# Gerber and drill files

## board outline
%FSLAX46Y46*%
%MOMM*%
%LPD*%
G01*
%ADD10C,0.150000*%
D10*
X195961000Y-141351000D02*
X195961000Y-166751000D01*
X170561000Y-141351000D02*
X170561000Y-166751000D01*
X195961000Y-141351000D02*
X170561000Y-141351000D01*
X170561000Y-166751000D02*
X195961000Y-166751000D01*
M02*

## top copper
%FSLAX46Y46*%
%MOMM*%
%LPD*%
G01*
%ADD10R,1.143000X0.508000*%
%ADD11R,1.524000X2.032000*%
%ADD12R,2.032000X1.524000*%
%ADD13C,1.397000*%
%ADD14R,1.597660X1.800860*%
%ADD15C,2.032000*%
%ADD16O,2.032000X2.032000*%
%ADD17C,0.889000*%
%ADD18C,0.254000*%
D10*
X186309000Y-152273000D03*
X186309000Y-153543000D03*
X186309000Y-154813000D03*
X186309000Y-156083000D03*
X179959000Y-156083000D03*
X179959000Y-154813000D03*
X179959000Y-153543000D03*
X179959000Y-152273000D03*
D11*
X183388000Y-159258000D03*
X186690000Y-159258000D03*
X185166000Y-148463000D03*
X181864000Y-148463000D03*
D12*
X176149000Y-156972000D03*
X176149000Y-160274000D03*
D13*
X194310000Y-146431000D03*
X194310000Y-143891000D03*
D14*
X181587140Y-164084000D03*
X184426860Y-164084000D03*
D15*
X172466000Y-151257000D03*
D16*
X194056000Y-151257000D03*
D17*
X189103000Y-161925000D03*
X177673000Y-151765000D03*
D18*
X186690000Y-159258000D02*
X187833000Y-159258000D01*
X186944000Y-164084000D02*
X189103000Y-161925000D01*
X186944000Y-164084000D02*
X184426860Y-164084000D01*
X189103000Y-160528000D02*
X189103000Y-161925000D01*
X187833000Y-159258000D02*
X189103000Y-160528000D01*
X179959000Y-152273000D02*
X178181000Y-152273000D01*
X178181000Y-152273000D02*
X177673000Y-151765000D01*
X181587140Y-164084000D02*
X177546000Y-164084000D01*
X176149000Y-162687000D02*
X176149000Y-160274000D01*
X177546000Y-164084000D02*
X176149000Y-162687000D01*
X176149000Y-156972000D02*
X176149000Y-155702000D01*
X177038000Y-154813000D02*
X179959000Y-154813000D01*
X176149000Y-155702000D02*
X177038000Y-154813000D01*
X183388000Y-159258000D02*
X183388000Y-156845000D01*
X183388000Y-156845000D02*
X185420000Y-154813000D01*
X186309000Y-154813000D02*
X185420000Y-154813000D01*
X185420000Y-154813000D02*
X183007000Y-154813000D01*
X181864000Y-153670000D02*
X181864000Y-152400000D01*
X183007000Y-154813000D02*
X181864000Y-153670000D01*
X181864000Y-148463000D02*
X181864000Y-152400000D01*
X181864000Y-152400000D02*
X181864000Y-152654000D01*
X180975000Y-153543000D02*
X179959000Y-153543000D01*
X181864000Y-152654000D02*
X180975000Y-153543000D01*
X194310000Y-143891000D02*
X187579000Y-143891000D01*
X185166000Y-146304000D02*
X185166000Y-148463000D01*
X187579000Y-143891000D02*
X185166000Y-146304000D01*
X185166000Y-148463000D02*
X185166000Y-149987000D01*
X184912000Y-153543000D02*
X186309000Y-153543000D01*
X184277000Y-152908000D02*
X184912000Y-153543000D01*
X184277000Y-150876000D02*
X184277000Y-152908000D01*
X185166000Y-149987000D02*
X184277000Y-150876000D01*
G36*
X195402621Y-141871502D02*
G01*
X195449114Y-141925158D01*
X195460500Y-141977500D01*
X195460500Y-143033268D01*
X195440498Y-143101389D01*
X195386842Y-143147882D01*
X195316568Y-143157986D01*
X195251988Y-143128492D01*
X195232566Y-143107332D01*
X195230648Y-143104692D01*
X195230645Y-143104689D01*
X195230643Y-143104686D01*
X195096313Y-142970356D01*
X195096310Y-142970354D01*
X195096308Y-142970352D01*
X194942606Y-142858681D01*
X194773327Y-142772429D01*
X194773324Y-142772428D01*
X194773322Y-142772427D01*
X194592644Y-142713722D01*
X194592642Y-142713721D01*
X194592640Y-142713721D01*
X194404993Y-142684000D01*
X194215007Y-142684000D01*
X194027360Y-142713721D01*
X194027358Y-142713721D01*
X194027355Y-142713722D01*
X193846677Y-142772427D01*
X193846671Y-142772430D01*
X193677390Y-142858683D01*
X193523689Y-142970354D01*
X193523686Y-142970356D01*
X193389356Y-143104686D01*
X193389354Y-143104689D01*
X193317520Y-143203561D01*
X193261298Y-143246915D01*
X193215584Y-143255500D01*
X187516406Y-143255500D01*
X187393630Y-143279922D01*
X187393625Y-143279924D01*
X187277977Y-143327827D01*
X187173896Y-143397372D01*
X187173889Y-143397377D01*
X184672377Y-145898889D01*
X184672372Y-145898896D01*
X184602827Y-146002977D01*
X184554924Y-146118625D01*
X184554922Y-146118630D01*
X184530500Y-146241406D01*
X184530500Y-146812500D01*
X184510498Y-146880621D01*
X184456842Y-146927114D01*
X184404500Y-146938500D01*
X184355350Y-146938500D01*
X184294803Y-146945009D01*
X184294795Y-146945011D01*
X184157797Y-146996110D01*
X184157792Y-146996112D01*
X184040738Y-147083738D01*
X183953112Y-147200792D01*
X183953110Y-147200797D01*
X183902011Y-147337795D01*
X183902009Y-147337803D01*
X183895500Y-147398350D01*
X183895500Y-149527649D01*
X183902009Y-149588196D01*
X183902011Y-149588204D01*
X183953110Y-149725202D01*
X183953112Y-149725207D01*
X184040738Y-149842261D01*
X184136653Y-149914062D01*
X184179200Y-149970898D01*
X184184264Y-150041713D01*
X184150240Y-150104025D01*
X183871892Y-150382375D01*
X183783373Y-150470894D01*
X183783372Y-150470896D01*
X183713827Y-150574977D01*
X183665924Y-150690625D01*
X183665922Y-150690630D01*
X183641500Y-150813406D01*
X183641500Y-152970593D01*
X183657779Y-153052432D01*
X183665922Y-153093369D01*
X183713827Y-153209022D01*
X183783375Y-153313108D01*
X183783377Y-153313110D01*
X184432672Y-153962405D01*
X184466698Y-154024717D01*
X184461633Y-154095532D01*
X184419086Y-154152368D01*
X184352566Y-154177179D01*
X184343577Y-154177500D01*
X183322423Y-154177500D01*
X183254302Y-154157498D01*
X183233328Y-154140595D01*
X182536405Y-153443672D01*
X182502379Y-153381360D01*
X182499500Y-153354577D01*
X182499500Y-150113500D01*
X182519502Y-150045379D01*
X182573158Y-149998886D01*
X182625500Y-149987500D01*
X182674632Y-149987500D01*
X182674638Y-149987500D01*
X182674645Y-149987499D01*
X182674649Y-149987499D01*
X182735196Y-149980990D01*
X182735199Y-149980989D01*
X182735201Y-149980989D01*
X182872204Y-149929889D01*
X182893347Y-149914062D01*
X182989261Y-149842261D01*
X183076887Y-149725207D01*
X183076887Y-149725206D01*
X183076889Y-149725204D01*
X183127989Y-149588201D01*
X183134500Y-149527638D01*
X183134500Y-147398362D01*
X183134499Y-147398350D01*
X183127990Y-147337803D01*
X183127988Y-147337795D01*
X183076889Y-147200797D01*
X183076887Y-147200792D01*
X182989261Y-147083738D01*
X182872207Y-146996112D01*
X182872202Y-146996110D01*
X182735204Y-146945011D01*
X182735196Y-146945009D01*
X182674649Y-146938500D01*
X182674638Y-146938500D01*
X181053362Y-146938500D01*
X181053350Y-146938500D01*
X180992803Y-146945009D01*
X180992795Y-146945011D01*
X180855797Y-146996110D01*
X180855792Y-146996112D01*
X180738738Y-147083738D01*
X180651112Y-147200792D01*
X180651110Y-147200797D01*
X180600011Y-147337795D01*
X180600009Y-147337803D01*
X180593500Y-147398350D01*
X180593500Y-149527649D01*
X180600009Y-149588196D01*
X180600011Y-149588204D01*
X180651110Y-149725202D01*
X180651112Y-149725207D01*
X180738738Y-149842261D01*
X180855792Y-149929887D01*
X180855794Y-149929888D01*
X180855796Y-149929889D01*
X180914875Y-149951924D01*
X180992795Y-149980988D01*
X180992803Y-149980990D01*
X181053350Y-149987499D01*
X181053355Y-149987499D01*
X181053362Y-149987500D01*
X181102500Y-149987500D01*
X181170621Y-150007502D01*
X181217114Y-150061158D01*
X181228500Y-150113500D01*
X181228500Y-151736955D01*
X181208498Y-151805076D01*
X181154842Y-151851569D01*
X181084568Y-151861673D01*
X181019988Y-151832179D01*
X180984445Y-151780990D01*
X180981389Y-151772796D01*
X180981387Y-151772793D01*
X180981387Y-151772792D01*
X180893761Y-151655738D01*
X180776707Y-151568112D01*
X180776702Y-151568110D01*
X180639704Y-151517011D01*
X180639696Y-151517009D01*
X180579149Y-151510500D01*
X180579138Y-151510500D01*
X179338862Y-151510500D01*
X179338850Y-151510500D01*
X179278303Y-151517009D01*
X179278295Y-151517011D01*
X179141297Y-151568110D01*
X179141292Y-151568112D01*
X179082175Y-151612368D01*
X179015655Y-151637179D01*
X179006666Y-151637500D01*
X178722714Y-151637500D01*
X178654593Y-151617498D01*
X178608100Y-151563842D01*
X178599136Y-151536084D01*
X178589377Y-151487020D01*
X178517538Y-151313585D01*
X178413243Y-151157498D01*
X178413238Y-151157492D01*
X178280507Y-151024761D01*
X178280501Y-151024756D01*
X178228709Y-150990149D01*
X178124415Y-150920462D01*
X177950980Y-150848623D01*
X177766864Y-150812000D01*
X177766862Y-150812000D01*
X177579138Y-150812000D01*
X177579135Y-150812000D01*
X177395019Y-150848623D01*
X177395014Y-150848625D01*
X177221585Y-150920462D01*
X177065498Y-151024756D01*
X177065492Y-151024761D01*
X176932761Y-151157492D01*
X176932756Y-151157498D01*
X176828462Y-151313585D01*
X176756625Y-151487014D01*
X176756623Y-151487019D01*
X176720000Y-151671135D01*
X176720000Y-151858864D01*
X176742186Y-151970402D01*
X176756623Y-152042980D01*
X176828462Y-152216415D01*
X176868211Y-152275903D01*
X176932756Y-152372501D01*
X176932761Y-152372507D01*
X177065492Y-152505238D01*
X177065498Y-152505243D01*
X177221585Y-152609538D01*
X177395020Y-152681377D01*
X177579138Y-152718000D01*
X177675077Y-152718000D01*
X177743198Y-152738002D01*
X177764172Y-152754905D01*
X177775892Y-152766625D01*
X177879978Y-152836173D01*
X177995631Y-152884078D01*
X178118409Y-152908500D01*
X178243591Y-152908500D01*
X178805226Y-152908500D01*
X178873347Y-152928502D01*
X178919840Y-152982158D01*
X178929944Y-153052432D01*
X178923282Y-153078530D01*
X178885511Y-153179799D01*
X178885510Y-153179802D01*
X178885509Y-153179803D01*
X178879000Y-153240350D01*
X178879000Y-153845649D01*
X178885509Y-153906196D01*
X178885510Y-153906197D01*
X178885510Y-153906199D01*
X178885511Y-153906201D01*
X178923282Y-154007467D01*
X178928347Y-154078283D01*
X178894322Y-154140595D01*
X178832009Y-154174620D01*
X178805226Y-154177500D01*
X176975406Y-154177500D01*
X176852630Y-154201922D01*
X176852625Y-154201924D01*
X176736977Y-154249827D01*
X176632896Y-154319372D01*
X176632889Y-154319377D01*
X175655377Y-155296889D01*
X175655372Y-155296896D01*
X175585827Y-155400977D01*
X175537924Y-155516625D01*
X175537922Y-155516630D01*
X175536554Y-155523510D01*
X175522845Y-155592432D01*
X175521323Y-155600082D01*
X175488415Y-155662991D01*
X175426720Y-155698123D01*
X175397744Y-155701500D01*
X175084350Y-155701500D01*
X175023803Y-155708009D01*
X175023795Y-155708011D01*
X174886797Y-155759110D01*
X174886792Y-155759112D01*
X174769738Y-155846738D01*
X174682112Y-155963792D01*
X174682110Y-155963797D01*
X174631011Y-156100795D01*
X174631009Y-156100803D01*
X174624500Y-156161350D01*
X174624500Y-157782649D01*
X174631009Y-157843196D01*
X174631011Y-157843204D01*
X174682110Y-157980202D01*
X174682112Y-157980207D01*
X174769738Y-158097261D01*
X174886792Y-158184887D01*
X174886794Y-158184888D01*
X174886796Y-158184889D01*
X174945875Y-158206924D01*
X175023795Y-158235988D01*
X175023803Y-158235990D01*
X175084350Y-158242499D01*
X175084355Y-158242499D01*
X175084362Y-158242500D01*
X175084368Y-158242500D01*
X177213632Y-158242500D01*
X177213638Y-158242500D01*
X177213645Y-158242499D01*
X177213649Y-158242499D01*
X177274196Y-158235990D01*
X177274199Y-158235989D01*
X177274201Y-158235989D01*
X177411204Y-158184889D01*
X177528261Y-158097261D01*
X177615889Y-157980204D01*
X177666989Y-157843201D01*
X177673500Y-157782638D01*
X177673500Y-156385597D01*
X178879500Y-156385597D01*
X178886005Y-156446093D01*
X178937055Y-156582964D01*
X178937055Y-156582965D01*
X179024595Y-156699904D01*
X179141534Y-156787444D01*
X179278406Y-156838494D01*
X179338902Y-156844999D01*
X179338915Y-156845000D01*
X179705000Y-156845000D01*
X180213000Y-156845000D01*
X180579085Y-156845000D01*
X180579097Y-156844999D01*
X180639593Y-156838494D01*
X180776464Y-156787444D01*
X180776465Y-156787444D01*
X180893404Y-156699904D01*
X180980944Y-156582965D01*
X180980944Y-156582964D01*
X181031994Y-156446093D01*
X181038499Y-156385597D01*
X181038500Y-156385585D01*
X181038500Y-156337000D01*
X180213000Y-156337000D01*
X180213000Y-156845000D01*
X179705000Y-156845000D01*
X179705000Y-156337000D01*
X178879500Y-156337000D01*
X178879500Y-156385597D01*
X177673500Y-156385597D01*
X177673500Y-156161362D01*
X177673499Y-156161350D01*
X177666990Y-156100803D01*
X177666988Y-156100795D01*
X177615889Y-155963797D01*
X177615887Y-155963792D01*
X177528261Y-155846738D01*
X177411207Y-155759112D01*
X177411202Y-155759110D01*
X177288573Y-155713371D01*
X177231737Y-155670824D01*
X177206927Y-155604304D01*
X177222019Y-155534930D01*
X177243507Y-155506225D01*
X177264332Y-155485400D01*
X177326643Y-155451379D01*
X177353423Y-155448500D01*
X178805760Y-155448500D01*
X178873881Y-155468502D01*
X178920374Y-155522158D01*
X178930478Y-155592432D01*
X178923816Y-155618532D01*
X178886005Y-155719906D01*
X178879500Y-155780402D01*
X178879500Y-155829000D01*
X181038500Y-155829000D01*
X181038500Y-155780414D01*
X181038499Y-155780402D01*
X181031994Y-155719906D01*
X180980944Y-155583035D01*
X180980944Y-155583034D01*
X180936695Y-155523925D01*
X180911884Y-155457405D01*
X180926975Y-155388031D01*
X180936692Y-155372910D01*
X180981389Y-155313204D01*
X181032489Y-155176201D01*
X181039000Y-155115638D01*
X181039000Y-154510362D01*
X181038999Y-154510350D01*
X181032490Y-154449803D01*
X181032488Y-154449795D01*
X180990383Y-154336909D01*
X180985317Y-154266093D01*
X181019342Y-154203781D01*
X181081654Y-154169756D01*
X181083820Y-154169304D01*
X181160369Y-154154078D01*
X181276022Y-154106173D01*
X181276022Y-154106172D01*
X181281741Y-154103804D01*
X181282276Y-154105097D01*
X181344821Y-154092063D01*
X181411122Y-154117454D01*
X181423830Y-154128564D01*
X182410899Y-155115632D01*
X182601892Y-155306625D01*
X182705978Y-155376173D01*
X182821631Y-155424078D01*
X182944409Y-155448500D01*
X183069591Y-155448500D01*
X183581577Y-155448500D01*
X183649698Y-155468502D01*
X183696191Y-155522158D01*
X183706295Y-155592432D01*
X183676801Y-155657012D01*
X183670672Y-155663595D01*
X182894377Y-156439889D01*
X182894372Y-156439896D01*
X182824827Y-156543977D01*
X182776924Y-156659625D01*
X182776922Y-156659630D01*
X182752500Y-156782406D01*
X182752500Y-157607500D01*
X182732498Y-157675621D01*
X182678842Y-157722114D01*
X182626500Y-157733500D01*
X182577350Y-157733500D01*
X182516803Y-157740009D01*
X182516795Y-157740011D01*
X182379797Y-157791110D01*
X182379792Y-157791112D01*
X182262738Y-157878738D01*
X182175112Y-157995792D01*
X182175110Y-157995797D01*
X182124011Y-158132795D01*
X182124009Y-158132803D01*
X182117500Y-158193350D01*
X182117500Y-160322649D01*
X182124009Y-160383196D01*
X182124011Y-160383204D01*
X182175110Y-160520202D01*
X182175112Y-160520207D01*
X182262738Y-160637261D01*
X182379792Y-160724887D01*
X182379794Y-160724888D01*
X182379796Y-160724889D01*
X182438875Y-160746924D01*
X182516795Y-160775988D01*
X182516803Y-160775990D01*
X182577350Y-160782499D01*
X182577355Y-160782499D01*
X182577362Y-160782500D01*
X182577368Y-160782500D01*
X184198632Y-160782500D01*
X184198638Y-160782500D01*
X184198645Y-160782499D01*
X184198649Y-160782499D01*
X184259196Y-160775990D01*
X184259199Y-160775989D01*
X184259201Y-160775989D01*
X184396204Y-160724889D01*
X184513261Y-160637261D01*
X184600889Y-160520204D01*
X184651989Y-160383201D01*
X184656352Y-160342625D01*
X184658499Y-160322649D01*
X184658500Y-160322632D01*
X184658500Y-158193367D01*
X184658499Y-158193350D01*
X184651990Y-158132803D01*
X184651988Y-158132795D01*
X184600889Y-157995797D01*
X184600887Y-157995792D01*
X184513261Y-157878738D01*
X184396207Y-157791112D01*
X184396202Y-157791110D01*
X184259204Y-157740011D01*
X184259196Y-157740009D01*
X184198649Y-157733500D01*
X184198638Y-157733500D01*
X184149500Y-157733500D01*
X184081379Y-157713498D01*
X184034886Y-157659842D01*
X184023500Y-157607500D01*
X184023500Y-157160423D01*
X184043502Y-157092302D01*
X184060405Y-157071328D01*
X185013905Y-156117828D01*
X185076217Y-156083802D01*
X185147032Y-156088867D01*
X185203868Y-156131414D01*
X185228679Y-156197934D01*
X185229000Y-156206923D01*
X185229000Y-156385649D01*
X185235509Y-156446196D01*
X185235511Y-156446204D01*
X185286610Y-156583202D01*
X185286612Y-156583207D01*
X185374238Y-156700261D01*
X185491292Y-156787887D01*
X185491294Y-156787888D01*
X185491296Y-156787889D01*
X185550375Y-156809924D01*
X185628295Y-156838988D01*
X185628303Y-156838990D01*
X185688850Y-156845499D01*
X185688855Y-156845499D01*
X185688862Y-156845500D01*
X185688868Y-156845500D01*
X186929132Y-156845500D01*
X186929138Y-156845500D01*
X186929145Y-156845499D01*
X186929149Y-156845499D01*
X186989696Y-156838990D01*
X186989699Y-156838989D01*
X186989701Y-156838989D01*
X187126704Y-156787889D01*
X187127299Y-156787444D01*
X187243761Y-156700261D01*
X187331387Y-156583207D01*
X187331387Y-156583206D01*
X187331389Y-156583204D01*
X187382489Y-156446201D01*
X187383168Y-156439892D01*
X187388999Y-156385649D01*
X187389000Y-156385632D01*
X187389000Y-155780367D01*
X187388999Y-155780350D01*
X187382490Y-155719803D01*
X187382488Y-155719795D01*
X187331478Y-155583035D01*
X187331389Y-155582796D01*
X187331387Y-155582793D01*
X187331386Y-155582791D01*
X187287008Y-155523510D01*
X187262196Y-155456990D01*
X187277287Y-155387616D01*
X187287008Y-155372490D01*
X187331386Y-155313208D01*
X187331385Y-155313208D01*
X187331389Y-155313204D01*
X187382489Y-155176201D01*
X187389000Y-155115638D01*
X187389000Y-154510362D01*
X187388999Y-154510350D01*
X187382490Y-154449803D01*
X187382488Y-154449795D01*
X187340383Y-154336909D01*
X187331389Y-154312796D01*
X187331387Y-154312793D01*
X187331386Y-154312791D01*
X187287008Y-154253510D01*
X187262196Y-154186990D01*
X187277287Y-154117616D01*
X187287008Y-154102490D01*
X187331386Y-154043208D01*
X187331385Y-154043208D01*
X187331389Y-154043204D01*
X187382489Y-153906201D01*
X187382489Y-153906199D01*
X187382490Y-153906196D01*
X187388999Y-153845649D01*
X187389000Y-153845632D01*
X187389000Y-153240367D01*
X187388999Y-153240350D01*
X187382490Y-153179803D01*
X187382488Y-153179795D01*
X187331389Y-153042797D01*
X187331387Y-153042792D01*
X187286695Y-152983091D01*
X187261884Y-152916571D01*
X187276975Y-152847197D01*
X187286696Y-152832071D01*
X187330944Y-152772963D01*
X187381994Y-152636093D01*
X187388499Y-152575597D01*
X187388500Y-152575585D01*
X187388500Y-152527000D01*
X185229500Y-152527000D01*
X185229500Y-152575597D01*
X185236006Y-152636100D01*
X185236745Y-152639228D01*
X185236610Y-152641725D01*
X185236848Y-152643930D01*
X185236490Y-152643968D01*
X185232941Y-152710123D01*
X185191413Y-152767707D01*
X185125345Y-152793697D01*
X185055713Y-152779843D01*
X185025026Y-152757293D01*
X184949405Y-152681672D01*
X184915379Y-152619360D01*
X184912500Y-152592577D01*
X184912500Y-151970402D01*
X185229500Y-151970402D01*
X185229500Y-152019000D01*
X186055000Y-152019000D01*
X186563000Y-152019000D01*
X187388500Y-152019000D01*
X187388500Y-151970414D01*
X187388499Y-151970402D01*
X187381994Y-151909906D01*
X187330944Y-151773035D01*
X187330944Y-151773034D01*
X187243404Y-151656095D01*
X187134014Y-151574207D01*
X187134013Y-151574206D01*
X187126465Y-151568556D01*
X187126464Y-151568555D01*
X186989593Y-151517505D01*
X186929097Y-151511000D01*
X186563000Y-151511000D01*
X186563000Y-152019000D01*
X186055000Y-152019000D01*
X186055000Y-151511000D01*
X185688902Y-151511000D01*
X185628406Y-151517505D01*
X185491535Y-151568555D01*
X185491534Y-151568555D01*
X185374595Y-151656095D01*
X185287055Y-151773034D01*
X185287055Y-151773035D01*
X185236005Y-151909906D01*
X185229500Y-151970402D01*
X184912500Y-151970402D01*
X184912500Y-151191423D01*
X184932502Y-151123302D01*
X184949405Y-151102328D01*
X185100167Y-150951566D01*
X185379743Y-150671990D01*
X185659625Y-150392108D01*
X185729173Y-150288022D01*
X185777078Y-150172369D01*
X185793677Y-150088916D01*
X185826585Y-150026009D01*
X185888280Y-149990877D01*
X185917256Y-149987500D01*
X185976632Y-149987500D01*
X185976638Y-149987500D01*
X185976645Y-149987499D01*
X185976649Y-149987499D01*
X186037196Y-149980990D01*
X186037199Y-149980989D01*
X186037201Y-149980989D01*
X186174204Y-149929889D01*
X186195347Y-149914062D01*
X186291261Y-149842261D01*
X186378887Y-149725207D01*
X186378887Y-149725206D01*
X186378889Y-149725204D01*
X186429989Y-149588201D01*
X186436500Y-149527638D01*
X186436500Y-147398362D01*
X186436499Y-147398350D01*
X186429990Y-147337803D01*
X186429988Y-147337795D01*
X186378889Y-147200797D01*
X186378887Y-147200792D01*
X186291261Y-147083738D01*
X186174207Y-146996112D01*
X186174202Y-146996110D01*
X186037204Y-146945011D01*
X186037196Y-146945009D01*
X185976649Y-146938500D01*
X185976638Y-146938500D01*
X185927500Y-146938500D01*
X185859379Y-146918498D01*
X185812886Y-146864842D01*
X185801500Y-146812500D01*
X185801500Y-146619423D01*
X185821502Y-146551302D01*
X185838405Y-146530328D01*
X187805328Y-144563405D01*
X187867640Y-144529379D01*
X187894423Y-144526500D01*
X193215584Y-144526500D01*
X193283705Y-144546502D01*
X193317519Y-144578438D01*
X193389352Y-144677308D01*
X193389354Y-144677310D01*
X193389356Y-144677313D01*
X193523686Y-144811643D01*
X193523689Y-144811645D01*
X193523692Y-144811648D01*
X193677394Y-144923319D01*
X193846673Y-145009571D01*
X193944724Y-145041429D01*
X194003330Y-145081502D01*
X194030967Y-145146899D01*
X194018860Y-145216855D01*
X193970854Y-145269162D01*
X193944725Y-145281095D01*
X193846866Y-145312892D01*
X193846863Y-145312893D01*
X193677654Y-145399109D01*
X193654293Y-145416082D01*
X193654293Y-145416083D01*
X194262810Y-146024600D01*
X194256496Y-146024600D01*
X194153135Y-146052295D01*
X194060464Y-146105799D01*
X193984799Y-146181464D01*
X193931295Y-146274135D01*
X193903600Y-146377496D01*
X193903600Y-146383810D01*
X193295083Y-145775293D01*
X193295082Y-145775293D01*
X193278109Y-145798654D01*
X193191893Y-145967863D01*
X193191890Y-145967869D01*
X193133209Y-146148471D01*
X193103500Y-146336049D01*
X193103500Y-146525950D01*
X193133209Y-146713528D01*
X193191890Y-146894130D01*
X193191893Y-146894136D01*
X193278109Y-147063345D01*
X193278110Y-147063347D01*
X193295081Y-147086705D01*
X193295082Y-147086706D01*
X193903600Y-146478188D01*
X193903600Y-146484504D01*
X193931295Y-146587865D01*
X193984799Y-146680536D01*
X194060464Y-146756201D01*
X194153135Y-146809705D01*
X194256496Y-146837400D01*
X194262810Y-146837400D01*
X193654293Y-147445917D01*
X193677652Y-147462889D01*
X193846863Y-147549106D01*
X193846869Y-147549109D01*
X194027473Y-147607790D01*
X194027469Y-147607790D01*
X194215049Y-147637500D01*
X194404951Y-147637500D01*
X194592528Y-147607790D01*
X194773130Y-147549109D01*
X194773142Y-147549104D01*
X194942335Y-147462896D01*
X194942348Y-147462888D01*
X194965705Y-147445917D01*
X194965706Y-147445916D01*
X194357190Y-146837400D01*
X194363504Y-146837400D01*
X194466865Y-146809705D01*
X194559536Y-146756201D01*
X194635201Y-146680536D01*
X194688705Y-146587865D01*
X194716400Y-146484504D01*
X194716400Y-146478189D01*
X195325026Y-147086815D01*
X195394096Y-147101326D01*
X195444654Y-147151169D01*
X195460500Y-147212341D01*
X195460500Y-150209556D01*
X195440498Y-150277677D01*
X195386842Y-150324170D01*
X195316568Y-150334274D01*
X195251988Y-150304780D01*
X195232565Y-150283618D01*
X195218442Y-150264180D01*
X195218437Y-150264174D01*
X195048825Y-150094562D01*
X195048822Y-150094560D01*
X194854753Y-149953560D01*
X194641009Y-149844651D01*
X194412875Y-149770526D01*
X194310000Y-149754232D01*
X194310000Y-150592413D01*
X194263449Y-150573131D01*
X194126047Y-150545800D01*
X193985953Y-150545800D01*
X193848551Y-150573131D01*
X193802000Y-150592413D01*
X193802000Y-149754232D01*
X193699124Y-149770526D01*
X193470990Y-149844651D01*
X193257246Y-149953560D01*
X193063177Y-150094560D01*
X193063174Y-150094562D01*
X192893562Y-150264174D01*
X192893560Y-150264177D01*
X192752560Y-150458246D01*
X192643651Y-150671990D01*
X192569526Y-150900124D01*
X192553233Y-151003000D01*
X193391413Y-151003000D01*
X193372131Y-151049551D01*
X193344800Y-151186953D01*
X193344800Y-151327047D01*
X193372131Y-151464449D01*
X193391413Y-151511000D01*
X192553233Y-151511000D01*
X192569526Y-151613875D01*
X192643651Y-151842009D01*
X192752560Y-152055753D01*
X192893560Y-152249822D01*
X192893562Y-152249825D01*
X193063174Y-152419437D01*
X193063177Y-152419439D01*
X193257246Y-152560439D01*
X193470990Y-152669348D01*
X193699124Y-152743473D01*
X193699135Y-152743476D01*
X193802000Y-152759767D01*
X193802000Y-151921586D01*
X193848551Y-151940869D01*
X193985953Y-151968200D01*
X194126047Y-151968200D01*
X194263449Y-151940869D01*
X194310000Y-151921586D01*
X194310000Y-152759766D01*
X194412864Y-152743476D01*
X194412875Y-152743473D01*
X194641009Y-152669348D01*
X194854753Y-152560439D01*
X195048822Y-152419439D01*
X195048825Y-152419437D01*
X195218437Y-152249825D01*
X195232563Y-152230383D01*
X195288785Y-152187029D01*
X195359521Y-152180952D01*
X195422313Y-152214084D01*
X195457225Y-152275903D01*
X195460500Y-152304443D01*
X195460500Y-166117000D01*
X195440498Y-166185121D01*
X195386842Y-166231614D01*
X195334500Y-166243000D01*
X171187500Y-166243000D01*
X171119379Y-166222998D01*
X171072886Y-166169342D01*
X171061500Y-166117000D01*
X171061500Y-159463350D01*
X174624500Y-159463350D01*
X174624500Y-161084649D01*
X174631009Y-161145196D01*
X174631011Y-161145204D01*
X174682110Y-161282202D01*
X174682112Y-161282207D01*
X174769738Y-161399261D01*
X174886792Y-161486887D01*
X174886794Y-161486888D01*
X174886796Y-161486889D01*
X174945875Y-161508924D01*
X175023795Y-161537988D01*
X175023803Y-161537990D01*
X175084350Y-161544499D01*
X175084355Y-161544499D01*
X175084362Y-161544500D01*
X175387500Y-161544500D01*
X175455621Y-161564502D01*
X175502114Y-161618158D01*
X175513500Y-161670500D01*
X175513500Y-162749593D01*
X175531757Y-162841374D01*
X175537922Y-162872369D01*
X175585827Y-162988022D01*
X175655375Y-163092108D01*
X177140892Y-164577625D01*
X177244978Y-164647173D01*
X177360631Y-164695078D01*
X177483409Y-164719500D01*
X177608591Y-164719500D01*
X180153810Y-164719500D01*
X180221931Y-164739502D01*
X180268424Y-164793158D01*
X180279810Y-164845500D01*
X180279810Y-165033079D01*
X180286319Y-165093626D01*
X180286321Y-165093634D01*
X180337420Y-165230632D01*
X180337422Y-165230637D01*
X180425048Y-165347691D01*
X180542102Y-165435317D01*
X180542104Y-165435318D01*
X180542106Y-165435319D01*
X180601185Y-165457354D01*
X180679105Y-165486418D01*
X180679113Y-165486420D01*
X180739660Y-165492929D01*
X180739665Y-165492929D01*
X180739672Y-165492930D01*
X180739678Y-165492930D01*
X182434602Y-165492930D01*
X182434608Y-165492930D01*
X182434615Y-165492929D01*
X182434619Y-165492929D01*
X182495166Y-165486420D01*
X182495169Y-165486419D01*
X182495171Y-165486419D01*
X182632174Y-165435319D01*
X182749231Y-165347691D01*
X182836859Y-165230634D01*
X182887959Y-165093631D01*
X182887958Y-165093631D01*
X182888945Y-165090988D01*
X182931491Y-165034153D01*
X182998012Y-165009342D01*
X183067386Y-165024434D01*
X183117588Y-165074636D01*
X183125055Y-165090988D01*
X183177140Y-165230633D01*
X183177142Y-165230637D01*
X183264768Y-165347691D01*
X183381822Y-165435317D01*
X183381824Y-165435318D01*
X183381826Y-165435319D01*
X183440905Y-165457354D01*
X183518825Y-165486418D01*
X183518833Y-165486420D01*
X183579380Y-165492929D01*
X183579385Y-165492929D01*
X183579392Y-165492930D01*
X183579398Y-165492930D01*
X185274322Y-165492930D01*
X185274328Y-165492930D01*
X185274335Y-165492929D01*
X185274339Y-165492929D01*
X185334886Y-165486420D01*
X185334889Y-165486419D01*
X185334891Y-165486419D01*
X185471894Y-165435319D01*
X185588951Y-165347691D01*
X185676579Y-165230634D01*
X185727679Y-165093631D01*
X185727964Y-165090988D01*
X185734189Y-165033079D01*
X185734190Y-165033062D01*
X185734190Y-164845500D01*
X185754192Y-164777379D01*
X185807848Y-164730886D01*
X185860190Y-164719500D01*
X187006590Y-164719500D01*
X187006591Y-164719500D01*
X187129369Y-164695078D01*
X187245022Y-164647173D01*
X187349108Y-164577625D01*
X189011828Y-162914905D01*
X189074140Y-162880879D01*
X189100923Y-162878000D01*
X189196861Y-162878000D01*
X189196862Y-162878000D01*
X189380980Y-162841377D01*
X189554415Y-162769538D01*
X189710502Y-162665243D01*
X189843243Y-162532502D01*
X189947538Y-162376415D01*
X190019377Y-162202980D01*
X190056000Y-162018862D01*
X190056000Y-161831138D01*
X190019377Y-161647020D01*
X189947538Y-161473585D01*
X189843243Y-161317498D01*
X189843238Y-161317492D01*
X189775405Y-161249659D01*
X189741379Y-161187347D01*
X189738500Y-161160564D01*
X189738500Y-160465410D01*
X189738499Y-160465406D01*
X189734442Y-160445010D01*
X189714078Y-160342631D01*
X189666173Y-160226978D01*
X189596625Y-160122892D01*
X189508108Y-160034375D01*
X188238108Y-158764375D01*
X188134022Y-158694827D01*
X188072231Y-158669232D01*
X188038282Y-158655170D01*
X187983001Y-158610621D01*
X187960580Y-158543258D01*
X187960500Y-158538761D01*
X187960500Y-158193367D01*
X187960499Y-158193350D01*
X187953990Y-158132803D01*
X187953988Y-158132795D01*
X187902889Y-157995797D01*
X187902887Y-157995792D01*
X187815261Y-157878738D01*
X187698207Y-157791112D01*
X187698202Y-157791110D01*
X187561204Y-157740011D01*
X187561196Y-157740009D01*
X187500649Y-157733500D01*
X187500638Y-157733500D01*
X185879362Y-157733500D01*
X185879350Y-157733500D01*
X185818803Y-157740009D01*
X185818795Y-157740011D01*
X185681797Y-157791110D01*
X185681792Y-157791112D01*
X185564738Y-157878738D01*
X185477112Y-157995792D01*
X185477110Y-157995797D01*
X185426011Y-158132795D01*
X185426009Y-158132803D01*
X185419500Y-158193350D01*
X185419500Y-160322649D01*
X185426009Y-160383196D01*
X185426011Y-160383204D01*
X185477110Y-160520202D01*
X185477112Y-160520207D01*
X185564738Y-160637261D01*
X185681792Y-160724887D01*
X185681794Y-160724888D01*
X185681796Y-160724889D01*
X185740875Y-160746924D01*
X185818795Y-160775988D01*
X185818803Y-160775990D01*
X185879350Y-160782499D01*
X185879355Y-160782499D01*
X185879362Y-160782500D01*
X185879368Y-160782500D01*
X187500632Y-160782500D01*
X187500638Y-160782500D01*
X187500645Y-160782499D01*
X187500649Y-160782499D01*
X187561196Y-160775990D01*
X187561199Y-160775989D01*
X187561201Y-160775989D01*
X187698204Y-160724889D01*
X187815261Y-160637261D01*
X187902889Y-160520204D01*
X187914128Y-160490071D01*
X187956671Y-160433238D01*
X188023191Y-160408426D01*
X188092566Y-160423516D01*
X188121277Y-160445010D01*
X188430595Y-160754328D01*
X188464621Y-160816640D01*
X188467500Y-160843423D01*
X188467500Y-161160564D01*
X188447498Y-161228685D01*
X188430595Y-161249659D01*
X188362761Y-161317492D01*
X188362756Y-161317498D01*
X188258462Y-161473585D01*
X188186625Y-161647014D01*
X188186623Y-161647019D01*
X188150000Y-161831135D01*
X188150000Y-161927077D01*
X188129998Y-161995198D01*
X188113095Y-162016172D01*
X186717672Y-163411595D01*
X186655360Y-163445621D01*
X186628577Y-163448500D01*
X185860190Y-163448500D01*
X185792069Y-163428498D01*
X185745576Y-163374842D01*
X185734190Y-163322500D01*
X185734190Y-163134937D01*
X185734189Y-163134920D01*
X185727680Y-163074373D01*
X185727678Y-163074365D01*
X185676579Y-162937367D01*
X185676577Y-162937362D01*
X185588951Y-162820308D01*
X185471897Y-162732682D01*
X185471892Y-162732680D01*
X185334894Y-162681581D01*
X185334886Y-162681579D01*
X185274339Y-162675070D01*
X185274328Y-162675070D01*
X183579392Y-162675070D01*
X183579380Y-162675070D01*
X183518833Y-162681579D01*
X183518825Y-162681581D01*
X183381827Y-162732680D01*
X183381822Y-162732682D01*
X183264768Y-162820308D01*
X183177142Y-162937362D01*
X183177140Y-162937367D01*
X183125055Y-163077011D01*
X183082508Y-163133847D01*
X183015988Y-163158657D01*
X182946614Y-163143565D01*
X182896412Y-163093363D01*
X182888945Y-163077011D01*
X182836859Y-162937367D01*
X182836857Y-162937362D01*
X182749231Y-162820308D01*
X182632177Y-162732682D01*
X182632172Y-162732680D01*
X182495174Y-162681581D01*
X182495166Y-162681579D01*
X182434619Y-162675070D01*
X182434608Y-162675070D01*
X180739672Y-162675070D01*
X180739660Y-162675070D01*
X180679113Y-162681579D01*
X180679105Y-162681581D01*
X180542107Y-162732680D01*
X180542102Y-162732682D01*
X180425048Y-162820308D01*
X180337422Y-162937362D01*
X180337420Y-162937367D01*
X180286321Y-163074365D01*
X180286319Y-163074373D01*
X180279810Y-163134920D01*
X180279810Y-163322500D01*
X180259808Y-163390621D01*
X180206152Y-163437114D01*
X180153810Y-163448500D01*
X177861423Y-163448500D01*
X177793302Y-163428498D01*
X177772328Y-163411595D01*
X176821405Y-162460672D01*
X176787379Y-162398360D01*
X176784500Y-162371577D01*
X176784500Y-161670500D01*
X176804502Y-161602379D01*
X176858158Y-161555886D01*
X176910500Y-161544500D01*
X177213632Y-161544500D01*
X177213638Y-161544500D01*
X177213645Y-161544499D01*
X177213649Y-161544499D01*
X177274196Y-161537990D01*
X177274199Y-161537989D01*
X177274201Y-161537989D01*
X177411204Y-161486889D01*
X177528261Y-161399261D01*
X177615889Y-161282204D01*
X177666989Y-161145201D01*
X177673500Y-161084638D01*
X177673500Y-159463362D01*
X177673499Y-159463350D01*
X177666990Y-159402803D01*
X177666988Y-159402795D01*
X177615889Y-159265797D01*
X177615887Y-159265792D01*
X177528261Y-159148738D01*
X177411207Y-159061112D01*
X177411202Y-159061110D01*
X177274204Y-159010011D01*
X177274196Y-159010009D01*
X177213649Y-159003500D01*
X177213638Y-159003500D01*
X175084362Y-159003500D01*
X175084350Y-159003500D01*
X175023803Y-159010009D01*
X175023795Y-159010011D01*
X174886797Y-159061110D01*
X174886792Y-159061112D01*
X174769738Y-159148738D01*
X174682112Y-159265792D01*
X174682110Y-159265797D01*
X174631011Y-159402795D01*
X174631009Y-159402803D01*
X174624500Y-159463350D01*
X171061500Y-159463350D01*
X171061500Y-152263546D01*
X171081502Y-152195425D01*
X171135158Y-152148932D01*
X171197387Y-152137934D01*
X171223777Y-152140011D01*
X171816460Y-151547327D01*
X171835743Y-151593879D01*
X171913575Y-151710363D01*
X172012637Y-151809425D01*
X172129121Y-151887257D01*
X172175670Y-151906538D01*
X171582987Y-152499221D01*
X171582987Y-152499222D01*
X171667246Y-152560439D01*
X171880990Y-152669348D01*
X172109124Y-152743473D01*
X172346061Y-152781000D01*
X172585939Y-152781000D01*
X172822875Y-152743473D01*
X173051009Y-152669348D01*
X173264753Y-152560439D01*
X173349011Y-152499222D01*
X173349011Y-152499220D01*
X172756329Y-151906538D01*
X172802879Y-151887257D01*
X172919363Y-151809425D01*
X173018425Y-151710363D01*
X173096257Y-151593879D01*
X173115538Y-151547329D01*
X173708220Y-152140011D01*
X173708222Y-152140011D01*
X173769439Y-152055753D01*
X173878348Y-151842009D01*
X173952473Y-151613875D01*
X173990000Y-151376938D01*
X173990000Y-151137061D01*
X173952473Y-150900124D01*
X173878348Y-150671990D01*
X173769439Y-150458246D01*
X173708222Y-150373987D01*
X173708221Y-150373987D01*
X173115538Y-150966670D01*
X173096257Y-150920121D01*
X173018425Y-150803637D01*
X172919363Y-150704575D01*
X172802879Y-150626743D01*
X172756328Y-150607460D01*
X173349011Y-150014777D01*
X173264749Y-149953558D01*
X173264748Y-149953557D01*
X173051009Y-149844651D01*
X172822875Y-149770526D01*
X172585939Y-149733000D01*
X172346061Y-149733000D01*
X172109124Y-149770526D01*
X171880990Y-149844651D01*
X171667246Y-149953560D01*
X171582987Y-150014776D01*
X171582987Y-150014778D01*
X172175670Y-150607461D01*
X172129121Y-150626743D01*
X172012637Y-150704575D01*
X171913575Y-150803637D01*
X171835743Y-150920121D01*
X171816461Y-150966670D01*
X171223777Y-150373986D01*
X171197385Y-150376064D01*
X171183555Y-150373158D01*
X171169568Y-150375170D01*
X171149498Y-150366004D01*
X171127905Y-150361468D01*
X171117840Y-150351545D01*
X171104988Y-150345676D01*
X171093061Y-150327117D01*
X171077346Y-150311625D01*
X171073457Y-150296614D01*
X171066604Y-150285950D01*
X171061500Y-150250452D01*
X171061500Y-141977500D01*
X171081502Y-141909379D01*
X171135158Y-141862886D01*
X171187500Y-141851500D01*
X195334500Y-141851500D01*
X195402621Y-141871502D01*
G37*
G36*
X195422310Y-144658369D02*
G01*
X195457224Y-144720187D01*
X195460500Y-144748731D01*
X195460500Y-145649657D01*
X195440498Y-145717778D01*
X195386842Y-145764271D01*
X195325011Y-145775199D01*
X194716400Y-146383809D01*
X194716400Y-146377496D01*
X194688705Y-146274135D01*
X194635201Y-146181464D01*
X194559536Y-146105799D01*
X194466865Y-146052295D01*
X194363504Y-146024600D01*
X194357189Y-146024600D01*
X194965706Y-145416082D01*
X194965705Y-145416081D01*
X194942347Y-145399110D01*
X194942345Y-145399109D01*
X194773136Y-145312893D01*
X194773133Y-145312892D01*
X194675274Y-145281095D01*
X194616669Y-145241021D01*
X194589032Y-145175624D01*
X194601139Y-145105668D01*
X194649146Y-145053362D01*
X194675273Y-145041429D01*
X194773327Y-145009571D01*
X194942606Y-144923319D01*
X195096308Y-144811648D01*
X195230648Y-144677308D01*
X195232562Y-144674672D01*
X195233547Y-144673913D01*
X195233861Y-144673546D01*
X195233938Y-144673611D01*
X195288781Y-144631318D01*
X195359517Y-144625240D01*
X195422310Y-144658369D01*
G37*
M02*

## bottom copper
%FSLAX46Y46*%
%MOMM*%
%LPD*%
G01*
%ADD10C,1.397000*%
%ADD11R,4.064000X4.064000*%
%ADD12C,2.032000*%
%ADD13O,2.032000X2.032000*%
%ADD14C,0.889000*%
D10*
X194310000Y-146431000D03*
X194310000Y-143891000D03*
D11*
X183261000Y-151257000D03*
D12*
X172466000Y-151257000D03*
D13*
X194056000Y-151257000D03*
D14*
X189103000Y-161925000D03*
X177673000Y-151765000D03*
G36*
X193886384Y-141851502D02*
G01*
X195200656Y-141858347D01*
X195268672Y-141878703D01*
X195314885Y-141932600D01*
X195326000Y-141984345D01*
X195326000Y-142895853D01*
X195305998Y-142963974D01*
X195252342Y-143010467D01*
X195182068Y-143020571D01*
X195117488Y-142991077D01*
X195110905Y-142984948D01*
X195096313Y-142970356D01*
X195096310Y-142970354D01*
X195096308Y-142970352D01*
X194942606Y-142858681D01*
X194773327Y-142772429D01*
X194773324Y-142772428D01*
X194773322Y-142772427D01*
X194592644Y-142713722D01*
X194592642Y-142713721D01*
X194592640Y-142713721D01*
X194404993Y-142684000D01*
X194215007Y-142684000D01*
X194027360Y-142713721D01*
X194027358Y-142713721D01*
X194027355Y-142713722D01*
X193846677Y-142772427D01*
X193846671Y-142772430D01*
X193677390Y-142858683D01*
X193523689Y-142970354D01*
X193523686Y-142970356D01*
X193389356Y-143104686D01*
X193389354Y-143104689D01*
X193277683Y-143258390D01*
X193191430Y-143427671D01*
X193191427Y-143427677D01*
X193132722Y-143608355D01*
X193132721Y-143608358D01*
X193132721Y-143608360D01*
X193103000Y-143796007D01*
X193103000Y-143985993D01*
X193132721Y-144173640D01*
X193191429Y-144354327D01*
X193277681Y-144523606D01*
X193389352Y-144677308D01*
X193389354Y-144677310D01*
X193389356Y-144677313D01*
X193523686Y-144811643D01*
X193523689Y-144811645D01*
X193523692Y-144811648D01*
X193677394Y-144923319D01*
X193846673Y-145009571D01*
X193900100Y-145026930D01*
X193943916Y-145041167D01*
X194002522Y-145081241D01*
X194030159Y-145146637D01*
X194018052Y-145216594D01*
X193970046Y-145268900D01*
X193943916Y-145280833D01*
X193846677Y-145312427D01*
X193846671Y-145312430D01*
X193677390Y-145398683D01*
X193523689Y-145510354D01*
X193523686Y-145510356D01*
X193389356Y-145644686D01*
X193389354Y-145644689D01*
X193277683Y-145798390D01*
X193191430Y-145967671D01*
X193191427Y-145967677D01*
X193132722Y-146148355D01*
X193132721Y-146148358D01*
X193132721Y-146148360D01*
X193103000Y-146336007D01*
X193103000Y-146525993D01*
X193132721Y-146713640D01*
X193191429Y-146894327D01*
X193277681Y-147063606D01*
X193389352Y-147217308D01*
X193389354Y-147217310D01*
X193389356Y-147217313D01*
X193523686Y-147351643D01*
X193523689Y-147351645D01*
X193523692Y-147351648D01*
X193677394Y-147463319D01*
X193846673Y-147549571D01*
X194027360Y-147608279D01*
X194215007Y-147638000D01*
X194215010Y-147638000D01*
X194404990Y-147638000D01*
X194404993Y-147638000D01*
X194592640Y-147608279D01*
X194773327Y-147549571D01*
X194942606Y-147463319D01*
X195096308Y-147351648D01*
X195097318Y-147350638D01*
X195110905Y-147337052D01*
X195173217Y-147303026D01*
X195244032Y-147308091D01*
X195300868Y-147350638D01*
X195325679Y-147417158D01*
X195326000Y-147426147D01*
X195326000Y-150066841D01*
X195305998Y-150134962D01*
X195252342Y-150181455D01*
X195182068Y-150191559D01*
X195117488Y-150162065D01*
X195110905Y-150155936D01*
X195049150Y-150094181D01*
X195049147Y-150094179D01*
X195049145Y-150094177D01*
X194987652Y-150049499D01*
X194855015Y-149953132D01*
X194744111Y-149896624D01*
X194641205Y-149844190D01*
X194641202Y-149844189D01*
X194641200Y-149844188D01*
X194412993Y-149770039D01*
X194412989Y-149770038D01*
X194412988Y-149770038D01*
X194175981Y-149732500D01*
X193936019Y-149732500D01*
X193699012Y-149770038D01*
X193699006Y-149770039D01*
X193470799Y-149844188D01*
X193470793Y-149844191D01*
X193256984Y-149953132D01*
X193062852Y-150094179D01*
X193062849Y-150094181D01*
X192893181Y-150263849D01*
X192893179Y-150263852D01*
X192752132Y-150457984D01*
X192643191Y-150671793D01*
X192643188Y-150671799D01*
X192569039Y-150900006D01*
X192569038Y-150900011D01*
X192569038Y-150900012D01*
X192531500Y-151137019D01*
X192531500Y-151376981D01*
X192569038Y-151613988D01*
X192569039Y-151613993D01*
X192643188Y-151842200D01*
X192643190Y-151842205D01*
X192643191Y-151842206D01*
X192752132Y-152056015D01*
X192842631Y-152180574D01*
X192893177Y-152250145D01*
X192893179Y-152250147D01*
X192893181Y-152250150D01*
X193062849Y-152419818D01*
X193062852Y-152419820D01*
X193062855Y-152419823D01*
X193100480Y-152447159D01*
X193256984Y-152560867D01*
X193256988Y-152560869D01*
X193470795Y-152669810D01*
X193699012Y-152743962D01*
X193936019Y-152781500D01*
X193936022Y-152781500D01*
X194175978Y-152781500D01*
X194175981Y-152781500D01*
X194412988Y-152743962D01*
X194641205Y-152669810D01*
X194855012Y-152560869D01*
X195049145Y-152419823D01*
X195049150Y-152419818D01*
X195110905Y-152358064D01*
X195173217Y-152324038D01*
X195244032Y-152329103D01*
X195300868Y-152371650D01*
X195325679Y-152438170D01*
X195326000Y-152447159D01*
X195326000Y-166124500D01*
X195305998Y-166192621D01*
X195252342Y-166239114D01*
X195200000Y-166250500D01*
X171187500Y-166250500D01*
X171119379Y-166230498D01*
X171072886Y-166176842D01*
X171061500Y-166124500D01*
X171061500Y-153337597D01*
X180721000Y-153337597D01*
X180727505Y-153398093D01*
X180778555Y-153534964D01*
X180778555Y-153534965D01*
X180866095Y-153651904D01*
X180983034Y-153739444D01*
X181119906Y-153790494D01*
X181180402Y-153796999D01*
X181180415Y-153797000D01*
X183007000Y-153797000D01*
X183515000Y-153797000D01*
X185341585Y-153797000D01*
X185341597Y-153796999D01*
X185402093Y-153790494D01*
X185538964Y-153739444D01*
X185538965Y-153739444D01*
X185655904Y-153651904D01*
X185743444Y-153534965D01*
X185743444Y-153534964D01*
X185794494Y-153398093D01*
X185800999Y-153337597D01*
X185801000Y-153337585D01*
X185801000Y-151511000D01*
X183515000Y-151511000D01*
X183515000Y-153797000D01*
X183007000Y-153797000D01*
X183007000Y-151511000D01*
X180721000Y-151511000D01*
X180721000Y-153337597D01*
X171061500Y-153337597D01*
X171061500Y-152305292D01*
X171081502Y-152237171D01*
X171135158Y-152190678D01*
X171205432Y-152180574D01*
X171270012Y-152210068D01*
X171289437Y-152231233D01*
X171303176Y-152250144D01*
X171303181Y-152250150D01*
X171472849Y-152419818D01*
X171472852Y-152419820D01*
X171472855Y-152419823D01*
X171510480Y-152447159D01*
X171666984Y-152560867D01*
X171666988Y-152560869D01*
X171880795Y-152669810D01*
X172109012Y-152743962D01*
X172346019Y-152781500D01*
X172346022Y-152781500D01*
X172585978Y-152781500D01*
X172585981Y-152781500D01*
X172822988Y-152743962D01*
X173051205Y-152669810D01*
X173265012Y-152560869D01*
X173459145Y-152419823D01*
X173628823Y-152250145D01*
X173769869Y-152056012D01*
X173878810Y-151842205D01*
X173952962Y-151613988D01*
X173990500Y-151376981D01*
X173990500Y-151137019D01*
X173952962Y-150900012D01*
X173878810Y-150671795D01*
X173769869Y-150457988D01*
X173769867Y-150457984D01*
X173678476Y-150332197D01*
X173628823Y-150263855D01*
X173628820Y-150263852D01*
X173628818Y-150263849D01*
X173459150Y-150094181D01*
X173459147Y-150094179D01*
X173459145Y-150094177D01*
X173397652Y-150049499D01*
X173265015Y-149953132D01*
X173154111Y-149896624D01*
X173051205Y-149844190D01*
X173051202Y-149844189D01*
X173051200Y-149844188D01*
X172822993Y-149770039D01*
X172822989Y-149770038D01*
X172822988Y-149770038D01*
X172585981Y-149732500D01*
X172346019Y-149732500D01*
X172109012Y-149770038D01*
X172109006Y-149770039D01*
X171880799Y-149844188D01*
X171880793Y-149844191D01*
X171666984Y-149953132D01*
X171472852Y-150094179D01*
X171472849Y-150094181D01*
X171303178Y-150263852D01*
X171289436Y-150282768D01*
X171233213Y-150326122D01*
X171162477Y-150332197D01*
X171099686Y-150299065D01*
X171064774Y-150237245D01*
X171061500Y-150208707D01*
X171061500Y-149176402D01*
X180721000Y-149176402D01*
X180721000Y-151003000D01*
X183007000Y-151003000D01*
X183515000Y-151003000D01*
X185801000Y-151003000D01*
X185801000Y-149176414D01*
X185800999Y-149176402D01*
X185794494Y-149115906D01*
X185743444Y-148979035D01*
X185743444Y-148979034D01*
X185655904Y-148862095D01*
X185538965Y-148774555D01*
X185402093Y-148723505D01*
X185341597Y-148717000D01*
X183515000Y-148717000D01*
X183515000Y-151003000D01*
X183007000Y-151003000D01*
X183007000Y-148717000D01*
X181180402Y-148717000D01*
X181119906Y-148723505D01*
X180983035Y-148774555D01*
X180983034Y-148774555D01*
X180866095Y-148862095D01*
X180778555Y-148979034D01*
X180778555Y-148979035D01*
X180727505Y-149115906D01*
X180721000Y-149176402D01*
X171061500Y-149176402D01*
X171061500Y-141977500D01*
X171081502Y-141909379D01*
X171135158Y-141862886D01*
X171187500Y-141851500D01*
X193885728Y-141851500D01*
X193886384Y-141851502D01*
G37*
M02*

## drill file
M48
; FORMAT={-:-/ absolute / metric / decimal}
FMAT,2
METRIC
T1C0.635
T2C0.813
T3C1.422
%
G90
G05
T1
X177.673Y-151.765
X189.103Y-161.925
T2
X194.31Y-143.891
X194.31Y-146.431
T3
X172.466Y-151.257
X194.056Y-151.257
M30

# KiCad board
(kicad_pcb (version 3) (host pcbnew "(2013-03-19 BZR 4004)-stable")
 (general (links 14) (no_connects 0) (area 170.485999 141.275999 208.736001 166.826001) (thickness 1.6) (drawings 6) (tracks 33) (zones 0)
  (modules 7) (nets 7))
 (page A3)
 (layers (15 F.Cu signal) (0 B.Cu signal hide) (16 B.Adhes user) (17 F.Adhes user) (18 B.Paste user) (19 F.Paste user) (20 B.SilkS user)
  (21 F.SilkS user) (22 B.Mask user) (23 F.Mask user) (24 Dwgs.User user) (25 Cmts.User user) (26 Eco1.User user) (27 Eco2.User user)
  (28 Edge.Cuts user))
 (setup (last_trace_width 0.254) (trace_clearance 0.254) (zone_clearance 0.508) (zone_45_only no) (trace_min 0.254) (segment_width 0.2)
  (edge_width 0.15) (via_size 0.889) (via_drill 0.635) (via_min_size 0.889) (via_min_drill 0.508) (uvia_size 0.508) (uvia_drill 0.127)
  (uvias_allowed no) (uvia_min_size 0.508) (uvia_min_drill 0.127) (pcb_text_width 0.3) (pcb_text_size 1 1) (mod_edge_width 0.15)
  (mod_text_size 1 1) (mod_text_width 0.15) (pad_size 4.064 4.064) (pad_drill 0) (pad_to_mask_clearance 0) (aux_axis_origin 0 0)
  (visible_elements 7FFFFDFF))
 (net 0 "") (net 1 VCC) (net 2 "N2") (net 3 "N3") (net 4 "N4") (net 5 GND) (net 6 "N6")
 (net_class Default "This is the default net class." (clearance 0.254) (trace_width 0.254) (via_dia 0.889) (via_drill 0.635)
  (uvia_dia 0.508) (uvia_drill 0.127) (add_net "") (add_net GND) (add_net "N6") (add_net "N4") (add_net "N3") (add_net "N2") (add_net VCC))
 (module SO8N (layer F.Cu) (at 183.134 154.178 270)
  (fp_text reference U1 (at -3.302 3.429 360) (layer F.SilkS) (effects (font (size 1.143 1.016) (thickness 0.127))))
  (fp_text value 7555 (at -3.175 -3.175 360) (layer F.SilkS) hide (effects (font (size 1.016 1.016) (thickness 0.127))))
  (pad 8 smd rect (at -1.905 -3.175 270) (size 0.508 1.143) (layers F.Cu F.Paste F.Mask) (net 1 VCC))
  (pad 7 smd rect (at -0.635 -3.175 270) (size 0.508 1.143) (layers F.Cu F.Paste F.Mask) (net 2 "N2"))
  (pad 6 smd rect (at 0.635 -3.175 270) (size 0.508 1.143) (layers F.Cu F.Paste F.Mask) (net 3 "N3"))
  (pad 5 smd rect (at 1.905 -3.175 270) (size 0.508 1.143) (layers F.Cu F.Paste F.Mask))
  (pad 4 smd rect (at 1.905 3.175 270) (size 0.508 1.143) (layers F.Cu F.Paste F.Mask) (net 1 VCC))
  (pad 3 smd rect (at 0.635 3.175 270) (size 0.508 1.143) (layers F.Cu F.Paste F.Mask) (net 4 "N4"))
  (pad 2 smd rect (at -0.635 3.175 270) (size 0.508 1.143) (layers F.Cu F.Paste F.Mask) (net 3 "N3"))
  (pad 1 smd rect (at -1.905 3.175 270) (size 0.508 1.143) (layers F.Cu F.Paste F.Mask) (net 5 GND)))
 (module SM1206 (layer F.Cu) (at 185.039 159.258)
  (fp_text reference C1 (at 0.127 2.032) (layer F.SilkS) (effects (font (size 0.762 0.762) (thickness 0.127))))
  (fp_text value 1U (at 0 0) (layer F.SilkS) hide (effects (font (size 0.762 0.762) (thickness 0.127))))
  (pad 1 smd rect (at -1.651 0) (size 1.524 2.032) (layers F.Cu F.Paste F.Mask) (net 3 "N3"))
  (pad 2 smd rect (at 1.651 0) (size 1.524 2.032) (layers F.Cu F.Paste F.Mask) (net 5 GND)))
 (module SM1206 (layer F.Cu) (at 183.515 148.463 180)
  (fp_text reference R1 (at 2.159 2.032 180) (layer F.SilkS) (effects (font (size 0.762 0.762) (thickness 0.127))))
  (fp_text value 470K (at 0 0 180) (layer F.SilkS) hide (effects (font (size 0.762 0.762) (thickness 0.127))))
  (pad 1 smd rect (at -1.651 0 180) (size 1.524 2.032) (layers F.Cu F.Paste F.Mask) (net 2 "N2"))
  (pad 2 smd rect (at 1.651 0 180) (size 1.524 2.032) (layers F.Cu F.Paste F.Mask) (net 3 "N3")))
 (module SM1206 (layer F.Cu) (at 176.149 158.623 270)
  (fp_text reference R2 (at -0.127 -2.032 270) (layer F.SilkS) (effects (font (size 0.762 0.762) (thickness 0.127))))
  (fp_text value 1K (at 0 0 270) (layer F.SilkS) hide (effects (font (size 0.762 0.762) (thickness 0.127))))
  (pad 1 smd rect (at -1.651 0 270) (size 1.524 2.032) (layers F.Cu F.Paste F.Mask) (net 4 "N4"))
  (pad 2 smd rect (at 1.651 0 270) (size 1.524 2.032) (layers F.Cu F.Paste F.Mask) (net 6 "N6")))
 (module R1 (layer F.Cu) (at 194.31 145.161 90) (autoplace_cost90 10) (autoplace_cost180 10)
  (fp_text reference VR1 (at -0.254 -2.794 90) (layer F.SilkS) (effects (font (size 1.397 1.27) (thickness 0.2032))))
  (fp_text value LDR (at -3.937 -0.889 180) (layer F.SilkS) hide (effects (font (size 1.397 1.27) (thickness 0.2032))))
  (pad 1 thru_hole circle (at -1.27 0 90) (size 1.397 1.397) (drill 0.812799) (layers *.Cu *.Mask F.SilkS) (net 1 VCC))
  (pad 2 thru_hole circle (at 1.27 0 90) (size 1.397 1.397) (drill 0.812799) (layers *.Cu *.Mask F.SilkS) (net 2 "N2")))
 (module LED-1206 (layer F.Cu) (at 183.007 164.084)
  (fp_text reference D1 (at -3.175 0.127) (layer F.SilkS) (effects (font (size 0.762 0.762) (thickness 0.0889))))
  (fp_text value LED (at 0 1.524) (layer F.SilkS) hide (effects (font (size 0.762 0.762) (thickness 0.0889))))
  (pad 1 smd rect (at -1.41986 0) (size 1.59766 1.80086) (layers F.Cu F.Paste F.Mask) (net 6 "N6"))
  (pad 2 smd rect (at 1.41986 0) (size 1.59766 1.80086) (layers F.Cu F.Paste F.Mask) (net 5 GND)))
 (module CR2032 (layer B.Cu) (at 183.261 151.257 180)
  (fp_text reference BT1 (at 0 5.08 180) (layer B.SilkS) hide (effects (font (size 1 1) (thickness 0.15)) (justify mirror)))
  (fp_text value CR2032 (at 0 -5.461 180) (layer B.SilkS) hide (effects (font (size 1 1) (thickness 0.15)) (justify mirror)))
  (pad 2 smd rect (at 0 0 180) (size 4.064 4.064) (layers B.Cu B.Paste B.Mask) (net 5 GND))
  (pad 1 thru_hole circle (at 10.795 0 180) (size 2.032 2.032) (drill 1.4224) (layers *.Cu *.Mask B.SilkS) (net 1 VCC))
  (pad 1 thru_hole oval (at -10.795 0 180) (size 2.032 2.032) (drill 1.4224) (layers *.Cu *.Mask B.SilkS) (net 1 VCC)))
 (gr_line (start 195.961 141.351) (end 195.961 166.751) (angle 90) (layer Edge.Cuts) (width 0.15))
 (gr_line (start 170.561 141.351) (end 170.561 166.751) (angle 90) (layer Edge.Cuts) (width 0.15))
 (gr_line (start 195.961 141.351) (end 170.561 141.351) (angle 90) (layer Edge.Cuts) (width 0.15))
 (gr_line (start 170.561 166.751) (end 195.961 166.751) (angle 90) (layer Edge.Cuts) (width 0.15))
 (segment (start 186.69 159.258) (end 187.833 159.258) (width 0.254) (layer F.Cu) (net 5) (status 400000))
 (segment (start 186.944 164.084) (end 189.103 161.925) (width 0.254) (layer F.Cu) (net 5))
 (via (at 189.103 161.925) (size 0.889) (layers F.Cu B.Cu) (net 5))
 (segment (start 186.944 164.084) (end 184.42686 164.084) (width 0.254) (layer F.Cu) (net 5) (status 800000))
 (segment (start 189.103 160.528) (end 189.103 161.925) (width 0.254) (layer F.Cu) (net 5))
 (segment (start 187.833 159.258) (end 189.103 160.528) (width 0.254) (layer F.Cu) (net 5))
 (segment (start 179.959 152.273) (end 178.181 152.273) (width 0.254) (layer F.Cu) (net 5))
 (via (at 177.673 151.765) (size 0.889) (layers F.Cu B.Cu) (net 5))
 (segment (start 178.181 152.273) (end 177.673 151.765) (width 0.254) (layer F.Cu) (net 5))
 (segment (start 181.58714 164.084) (end 177.546 164.084) (width 0.254) (layer F.Cu) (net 6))
 (segment (start 176.149 162.687) (end 176.149 160.274) (width 0.254) (layer F.Cu) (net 6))
 (segment (start 177.546 164.084) (end 176.149 162.687) (width 0.254) (layer F.Cu) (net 6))
 (segment (start 176.149 156.972) (end 176.149 155.702) (width 0.254) (layer F.Cu) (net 4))
 (segment (start 177.038 154.813) (end 179.959 154.813) (width 0.254) (layer F.Cu) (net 4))
 (segment (start 176.149 155.702) (end 177.038 154.813) (width 0.254) (layer F.Cu) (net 4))
 (segment (start 183.388 159.258) (end 183.388 156.845) (width 0.254) (layer F.Cu) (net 3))
 (segment (start 183.388 156.845) (end 185.42 154.813) (width 0.254) (layer F.Cu) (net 3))
 (segment (start 186.309 154.813) (end 185.42 154.813) (width 0.254) (layer F.Cu) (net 3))
 (segment (start 185.42 154.813) (end 183.007 154.813) (width 0.254) (layer F.Cu) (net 3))
 (segment (start 181.864 153.67) (end 181.864 152.4) (width 0.254) (layer F.Cu) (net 3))
 (segment (start 183.007 154.813) (end 181.864 153.67) (width 0.254) (layer F.Cu) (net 3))
 (segment (start 181.864 148.463) (end 181.864 152.4) (width 0.254) (layer F.Cu) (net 3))
 (segment (start 181.864 152.4) (end 181.864 152.654) (width 0.254) (layer F.Cu) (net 3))
 (segment (start 180.975 153.543) (end 179.959 153.543) (width 0.254) (layer F.Cu) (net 3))
 (segment (start 181.864 152.654) (end 180.975 153.543) (width 0.254) (layer F.Cu) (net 3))
 (segment (start 194.31 143.891) (end 187.579 143.891) (width 0.254) (layer F.Cu) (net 2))
 (segment (start 185.166 146.304) (end 185.166 148.463) (width 0.254) (layer F.Cu) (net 2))
 (segment (start 187.579 143.891) (end 185.166 146.304) (width 0.254) (layer F.Cu) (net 2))
 (segment (start 185.166 148.463) (end 185.166 149.987) (width 0.254) (layer F.Cu) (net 2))
 (segment (start 184.912 153.543) (end 186.309 153.543) (width 0.254) (layer F.Cu) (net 2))
 (segment (start 184.277 152.908) (end 184.912 153.543) (width 0.254) (layer F.Cu) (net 2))
 (segment (start 184.277 150.876) (end 184.277 152.908) (width 0.254) (layer F.Cu) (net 2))
 (segment (start 185.166 149.987) (end 184.277 150.876) (width 0.254) (layer F.Cu) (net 2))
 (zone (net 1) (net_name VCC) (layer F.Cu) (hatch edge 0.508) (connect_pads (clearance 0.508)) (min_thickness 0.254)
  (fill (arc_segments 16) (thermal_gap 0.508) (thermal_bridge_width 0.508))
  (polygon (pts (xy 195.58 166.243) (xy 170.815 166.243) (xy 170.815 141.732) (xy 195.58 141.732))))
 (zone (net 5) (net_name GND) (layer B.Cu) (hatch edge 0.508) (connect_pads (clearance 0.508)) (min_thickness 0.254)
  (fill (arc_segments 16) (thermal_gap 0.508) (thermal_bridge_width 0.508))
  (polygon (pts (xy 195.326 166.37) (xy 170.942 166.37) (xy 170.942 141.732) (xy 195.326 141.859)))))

